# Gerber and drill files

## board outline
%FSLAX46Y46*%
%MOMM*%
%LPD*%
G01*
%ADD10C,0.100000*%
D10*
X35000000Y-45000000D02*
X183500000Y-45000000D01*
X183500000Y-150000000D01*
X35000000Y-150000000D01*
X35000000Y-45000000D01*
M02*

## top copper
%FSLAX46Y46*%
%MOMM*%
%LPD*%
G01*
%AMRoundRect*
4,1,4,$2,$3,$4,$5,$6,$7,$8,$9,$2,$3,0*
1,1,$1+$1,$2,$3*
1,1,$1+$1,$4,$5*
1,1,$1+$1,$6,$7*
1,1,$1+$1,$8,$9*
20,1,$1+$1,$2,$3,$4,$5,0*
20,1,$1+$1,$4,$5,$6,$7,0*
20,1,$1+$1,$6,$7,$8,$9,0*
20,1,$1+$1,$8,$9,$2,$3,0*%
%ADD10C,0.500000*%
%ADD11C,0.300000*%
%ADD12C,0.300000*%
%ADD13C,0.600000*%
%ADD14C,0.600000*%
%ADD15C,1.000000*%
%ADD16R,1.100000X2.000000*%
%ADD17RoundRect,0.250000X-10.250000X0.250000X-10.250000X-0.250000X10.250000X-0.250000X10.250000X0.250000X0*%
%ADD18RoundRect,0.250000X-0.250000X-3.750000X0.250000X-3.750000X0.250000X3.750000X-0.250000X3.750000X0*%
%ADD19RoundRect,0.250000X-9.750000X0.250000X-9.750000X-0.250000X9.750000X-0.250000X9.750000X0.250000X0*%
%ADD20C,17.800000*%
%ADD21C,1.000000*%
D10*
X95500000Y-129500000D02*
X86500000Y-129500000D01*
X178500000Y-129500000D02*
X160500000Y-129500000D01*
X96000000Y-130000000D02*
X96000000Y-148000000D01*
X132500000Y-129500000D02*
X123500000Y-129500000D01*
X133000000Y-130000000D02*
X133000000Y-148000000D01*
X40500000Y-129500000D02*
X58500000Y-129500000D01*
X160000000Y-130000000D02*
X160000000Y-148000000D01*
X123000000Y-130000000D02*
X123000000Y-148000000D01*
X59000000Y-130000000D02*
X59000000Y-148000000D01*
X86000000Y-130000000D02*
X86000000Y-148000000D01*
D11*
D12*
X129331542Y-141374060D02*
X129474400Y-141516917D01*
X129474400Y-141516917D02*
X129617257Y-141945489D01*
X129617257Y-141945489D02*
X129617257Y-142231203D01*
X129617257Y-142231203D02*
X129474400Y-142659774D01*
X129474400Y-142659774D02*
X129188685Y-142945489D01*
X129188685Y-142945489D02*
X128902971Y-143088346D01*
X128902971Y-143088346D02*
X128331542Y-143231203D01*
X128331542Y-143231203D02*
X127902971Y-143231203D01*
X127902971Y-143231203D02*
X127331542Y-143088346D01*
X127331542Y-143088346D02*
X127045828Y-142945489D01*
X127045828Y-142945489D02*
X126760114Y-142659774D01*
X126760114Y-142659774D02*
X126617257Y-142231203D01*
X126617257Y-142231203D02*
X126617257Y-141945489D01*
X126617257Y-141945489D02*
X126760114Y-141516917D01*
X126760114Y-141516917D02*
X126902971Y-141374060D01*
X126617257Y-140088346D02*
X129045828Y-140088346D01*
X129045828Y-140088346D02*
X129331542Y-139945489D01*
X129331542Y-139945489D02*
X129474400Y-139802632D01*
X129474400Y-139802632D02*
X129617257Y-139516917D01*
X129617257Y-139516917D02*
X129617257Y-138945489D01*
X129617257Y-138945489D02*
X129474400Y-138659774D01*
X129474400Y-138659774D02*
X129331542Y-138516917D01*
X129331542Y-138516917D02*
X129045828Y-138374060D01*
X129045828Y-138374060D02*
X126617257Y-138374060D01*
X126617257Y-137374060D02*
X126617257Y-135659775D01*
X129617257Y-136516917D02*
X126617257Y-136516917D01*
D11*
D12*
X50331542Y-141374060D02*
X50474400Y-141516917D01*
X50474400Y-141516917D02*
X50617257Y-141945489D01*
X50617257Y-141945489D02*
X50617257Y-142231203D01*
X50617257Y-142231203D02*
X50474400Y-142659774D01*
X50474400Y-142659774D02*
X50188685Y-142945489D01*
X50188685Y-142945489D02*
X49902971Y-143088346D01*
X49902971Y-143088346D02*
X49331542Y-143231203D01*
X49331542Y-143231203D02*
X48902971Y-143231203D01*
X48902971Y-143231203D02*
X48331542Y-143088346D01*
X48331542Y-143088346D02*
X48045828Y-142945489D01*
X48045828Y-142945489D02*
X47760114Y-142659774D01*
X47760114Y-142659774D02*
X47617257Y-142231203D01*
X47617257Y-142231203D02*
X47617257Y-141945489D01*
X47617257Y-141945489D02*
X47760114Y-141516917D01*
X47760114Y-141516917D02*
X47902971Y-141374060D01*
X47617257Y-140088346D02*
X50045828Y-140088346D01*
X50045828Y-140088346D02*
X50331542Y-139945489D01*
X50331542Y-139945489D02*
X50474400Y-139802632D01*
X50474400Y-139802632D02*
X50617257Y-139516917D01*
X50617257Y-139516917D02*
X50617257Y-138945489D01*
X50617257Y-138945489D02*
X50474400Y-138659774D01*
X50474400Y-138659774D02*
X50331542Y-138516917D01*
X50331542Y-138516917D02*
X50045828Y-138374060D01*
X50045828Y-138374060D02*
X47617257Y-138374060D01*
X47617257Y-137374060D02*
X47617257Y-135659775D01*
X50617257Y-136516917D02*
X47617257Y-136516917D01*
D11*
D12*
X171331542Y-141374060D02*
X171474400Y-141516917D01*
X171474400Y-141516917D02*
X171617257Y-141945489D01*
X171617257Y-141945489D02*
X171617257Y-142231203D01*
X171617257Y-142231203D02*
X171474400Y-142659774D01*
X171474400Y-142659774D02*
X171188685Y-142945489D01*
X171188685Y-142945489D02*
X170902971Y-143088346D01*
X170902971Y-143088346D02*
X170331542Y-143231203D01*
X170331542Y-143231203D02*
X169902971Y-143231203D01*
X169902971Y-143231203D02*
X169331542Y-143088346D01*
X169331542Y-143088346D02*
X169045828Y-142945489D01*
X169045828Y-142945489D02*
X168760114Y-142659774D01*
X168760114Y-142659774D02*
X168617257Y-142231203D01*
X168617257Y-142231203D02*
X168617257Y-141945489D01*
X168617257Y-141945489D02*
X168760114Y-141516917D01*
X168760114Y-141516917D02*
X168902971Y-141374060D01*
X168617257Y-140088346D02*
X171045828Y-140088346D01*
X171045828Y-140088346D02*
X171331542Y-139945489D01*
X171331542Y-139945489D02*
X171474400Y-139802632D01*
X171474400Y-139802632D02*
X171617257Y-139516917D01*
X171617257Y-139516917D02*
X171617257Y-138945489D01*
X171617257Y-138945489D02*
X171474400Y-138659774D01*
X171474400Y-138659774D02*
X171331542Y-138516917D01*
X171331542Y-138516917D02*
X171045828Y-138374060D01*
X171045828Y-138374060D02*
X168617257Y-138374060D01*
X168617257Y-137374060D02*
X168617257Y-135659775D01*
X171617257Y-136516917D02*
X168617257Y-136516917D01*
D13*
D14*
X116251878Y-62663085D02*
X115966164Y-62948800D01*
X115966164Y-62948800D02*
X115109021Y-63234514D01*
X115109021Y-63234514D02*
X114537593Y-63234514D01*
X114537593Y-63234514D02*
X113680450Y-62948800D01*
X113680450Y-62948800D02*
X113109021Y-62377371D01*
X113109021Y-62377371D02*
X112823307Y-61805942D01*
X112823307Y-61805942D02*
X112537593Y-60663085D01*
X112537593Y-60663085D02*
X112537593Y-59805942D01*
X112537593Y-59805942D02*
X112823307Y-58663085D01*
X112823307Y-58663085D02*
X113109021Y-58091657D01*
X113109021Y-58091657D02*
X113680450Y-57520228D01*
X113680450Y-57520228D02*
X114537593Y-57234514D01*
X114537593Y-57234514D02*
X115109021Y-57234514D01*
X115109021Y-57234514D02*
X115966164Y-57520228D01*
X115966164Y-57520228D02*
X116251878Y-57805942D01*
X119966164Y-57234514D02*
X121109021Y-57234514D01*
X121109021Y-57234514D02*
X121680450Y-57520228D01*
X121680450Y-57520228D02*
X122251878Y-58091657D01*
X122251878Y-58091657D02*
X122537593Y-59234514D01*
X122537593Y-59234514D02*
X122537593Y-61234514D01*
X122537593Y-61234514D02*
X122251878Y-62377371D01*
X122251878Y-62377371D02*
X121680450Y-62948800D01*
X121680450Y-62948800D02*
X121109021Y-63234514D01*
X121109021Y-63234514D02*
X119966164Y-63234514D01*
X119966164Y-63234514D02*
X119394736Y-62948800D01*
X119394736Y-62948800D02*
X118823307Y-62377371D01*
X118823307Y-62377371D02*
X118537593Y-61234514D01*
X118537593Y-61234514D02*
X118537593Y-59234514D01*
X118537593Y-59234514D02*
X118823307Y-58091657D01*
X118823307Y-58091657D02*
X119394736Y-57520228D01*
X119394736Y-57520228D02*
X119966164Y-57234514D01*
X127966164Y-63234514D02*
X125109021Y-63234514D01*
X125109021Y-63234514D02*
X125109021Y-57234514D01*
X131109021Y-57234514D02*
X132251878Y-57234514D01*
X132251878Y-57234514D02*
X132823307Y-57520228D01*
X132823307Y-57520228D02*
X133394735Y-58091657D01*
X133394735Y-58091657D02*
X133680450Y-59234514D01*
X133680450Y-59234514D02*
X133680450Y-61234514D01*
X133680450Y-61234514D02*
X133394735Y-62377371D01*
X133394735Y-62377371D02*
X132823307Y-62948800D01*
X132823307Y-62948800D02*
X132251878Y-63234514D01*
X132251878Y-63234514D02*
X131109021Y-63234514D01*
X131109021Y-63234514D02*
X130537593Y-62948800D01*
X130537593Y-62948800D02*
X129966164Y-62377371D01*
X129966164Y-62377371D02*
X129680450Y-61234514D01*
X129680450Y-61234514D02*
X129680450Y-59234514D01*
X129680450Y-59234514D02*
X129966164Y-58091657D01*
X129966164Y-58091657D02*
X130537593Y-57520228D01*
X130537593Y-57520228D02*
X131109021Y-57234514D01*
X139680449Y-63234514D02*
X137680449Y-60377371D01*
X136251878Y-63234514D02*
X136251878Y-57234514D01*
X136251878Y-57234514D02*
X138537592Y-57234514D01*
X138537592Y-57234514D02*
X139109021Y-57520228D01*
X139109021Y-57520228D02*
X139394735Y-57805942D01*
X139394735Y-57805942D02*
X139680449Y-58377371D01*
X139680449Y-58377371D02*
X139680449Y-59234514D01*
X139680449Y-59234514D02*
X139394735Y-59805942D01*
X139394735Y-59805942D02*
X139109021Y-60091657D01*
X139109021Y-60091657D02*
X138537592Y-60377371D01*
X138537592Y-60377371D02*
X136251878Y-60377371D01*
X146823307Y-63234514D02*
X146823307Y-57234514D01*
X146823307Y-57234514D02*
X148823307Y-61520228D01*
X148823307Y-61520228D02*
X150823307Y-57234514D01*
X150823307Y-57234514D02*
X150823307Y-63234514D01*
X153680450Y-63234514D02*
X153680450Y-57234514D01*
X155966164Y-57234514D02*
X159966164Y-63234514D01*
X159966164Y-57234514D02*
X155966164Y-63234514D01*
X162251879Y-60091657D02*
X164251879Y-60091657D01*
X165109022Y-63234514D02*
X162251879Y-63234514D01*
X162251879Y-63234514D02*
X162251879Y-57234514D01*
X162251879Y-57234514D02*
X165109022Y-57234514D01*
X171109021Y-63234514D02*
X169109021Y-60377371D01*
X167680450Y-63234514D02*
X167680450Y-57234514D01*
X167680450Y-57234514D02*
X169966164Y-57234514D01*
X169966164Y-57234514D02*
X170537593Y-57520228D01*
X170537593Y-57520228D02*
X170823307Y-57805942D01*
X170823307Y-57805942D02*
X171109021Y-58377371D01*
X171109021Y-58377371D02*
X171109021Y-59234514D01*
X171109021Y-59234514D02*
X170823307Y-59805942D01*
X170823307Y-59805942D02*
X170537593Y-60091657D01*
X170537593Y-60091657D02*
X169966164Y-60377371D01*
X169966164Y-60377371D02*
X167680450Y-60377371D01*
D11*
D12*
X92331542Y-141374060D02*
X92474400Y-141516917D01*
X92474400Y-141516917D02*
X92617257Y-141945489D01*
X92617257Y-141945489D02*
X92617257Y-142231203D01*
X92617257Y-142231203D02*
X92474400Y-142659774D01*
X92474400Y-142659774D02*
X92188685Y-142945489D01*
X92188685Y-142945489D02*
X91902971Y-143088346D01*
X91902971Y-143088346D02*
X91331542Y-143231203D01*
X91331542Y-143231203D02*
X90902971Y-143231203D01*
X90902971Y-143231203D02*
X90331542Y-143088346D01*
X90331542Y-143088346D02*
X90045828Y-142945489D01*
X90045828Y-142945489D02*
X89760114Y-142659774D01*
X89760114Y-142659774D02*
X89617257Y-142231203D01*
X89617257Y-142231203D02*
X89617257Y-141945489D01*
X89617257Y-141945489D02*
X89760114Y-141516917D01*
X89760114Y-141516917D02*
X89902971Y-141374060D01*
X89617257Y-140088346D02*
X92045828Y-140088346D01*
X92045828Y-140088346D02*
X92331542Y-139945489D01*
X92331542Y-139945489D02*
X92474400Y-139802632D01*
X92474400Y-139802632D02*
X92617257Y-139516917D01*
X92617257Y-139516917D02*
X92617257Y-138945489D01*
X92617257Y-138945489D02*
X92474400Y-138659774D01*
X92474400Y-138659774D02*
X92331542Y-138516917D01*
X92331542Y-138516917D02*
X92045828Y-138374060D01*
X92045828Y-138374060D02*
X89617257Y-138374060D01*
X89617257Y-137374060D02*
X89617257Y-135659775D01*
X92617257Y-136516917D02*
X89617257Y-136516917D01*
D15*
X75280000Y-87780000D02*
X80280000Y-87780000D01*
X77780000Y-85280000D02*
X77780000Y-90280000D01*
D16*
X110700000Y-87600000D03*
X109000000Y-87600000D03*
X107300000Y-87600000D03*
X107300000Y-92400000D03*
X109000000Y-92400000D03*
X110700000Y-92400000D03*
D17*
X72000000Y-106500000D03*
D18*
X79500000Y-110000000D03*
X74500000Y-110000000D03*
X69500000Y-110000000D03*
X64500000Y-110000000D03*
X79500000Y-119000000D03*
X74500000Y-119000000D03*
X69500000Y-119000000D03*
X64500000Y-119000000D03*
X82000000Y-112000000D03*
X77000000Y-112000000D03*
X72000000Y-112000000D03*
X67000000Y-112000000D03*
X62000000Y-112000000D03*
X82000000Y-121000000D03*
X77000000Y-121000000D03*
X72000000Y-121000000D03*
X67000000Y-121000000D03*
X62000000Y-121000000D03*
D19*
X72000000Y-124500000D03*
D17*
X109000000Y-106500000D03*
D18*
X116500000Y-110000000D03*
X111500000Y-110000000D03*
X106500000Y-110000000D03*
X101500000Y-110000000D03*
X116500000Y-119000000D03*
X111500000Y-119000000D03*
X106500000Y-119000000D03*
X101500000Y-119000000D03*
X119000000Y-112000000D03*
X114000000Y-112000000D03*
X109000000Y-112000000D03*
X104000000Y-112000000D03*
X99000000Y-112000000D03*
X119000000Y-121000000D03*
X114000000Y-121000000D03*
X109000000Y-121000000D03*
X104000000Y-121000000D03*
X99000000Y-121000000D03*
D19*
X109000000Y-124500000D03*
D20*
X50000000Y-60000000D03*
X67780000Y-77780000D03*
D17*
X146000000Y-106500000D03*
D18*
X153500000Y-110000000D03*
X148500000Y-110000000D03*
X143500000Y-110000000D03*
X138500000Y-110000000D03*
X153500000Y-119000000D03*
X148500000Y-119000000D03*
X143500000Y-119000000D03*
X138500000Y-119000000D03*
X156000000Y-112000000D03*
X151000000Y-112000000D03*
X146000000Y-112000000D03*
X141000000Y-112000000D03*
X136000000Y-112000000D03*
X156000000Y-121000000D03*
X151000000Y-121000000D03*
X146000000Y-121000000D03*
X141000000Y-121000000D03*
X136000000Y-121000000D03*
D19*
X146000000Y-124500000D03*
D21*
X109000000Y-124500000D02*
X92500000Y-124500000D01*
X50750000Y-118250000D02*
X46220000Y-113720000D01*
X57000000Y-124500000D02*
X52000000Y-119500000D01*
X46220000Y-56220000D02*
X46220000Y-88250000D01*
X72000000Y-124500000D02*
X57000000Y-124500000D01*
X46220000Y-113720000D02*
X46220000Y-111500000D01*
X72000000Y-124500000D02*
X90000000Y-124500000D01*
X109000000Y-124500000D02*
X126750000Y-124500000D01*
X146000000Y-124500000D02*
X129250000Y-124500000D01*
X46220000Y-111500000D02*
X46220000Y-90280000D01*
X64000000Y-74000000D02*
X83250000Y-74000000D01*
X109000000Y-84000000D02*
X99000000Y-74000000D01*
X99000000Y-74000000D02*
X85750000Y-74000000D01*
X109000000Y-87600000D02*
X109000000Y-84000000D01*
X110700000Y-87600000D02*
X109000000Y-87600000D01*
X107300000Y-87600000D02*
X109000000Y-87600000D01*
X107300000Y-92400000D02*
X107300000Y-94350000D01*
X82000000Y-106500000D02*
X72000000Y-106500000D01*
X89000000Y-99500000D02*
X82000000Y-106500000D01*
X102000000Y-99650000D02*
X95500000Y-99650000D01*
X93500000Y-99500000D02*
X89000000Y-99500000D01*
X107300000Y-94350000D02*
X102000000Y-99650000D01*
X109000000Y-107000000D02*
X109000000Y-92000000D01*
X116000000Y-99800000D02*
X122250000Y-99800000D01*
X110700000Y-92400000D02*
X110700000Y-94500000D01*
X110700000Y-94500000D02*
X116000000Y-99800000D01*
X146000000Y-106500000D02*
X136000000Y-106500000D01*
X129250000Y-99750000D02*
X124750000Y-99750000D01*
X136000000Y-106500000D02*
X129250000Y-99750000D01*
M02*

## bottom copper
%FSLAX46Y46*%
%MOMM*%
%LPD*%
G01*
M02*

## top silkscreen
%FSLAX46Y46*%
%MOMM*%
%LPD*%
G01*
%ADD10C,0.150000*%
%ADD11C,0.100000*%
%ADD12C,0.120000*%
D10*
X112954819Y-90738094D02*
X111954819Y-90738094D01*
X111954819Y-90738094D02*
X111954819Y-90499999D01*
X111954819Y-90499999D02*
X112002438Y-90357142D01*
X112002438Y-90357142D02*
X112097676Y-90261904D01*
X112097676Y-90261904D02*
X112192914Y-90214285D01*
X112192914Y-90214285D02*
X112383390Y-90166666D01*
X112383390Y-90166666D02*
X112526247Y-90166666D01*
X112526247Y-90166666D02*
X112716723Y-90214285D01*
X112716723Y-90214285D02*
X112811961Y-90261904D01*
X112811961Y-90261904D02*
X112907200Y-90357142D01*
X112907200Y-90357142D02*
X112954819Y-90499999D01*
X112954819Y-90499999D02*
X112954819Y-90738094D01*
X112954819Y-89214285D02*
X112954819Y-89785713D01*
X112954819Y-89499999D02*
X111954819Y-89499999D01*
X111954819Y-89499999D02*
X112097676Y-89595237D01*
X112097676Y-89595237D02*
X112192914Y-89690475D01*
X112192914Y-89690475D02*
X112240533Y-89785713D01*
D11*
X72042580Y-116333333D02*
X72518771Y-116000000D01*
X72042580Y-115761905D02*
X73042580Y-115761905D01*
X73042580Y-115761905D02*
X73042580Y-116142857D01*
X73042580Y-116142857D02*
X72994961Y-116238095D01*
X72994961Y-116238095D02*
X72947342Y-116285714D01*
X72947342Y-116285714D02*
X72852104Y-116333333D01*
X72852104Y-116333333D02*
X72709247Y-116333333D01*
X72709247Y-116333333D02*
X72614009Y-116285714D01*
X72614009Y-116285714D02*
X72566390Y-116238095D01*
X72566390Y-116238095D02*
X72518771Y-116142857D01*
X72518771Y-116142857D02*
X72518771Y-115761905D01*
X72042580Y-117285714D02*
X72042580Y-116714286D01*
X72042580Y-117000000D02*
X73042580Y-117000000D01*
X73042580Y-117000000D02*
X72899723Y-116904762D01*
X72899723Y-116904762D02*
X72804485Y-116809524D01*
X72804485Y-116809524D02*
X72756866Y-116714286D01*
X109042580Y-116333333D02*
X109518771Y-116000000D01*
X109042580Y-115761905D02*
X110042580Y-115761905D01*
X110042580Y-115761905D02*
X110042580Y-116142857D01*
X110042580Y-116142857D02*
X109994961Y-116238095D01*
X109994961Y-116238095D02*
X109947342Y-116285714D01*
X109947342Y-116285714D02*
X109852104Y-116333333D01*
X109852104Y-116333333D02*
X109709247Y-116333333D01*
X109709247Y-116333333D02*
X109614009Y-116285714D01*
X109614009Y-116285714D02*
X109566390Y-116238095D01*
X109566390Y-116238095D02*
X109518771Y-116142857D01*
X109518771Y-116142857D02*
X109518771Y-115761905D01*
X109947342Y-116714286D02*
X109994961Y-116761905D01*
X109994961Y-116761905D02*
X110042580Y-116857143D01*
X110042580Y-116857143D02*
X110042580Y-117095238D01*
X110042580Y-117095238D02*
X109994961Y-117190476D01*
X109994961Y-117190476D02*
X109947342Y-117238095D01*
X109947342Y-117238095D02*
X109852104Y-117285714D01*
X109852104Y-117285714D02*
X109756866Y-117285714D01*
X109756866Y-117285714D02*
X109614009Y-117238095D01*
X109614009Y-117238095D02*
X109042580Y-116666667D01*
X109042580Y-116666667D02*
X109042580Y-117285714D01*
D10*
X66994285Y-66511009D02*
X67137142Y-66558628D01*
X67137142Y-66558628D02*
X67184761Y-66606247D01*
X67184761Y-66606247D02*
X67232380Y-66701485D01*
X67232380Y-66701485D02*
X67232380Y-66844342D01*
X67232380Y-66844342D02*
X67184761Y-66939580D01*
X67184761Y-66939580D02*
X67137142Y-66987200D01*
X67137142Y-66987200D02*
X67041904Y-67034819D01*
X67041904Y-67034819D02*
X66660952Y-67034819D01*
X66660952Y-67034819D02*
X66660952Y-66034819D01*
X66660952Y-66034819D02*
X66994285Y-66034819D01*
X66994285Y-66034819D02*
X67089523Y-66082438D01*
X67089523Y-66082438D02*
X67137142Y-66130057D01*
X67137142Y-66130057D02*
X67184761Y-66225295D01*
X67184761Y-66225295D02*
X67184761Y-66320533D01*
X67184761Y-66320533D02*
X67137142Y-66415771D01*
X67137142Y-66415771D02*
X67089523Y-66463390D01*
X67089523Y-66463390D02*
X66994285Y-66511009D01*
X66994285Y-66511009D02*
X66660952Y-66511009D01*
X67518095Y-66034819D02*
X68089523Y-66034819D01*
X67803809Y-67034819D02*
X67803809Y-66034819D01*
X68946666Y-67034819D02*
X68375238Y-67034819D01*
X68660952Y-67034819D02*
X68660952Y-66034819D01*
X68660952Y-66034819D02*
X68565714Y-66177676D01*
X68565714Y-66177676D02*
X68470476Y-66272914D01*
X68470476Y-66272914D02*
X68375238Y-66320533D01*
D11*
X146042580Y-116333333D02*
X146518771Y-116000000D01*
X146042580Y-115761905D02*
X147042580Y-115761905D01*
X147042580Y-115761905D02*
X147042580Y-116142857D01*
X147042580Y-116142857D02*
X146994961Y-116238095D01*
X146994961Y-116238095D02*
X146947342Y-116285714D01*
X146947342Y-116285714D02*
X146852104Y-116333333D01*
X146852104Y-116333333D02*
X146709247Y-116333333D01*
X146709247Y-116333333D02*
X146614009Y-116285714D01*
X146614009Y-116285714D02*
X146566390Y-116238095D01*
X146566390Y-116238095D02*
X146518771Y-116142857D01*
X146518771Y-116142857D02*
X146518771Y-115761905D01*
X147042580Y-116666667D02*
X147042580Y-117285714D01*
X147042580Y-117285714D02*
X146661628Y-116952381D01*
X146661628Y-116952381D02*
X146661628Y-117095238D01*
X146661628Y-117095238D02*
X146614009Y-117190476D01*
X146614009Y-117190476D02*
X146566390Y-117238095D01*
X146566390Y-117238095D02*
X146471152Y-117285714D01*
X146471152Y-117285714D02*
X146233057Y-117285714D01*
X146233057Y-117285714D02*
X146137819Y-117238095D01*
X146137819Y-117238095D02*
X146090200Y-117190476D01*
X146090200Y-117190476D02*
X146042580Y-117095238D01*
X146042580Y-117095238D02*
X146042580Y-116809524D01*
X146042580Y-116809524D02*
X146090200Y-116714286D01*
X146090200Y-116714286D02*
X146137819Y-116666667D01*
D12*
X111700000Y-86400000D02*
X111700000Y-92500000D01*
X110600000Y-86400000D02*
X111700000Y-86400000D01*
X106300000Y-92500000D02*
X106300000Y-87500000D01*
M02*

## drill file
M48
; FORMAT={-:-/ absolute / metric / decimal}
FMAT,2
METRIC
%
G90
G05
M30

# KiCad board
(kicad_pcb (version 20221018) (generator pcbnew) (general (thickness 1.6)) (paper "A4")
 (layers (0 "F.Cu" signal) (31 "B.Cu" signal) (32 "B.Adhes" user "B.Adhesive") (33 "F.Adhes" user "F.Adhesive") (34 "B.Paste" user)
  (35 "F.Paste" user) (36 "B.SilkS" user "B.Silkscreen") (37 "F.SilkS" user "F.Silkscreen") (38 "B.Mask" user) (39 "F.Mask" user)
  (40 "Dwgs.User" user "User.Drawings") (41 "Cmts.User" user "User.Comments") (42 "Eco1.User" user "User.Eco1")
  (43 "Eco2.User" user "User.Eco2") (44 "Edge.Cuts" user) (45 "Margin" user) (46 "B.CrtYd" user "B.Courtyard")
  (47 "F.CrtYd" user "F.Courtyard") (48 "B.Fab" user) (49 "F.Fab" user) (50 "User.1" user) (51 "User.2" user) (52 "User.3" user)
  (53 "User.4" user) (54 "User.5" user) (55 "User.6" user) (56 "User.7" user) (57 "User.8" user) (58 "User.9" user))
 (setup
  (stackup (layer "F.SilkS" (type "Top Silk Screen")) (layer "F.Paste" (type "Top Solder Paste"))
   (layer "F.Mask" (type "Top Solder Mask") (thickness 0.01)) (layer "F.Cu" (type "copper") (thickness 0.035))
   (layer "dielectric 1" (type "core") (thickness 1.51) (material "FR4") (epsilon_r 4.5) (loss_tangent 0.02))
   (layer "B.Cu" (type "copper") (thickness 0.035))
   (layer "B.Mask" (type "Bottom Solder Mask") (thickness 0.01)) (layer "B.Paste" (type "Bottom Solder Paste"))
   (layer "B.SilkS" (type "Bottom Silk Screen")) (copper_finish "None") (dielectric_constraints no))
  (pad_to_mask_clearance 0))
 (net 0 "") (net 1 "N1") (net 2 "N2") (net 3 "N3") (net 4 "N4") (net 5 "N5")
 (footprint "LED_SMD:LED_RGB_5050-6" (layer "F.Cu") (at 109 90 -90)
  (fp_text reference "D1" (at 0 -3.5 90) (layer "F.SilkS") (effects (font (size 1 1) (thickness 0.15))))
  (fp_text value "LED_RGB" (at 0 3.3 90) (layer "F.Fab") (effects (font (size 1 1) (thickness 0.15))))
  (fp_line (start -3.6 -2.7) (end 2.5 -2.7) (stroke (width 0.12) (type solid)) (layer "F.SilkS"))
  (fp_line (start -3.6 -1.6) (end -3.6 -2.7) (stroke (width 0.12) (type solid)) (layer "F.SilkS"))
  (fp_line (start 2.5 2.7) (end -2.5 2.7) (stroke (width 0.12) (type solid)) (layer "F.SilkS"))
  (pad "1" smd rect (at -2.4 -1.7) (size 1.1 2) (layers "F.Cu" "F.Paste" "F.Mask") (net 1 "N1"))
  (pad "2" smd rect (at -2.4 0) (size 1.1 2) (layers "F.Cu" "F.Paste" "F.Mask") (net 1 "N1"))
  (pad "3" smd rect (at -2.4 1.7) (size 1.1 2) (layers "F.Cu" "F.Paste" "F.Mask") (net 1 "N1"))
  (pad "4" smd rect (at 2.4 1.7) (size 1.1 2) (layers "F.Cu" "F.Paste" "F.Mask") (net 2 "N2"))
  (pad "5" smd rect (at 2.4 0) (size 1.1 2) (layers "F.Cu" "F.Paste" "F.Mask") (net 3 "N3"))
  (pad "6" smd rect (at 2.4 -1.7) (size 1.1 2) (layers "F.Cu" "F.Paste" "F.Mask") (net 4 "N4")))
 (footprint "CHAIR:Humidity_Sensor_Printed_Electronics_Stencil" (layer "F.Cu") (at 72 116.5 -90)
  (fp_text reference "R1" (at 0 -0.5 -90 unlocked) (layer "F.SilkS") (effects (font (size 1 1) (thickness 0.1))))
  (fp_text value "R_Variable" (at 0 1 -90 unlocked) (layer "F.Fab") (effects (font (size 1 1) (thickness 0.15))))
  (pad "1" smd roundrect (at -10 0 270) (size 1 21) (layers "F.Cu" "F.Paste" "F.Mask") (roundrect_rratio 0.25) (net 2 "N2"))
  (pad "1" smd roundrect (at -6.5 -7.5) (size 1 8) (layers "F.Cu" "F.Paste" "F.Mask") (roundrect_rratio 0.25) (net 2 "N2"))
  (pad "1" smd roundrect (at -6.5 -2.5) (size 1 8) (layers "F.Cu" "F.Paste" "F.Mask") (roundrect_rratio 0.25) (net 2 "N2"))
  (pad "1" smd roundrect (at -6.5 2.5) (size 1 8) (layers "F.Cu" "F.Paste" "F.Mask") (roundrect_rratio 0.25) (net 2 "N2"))
  (pad "1" smd roundrect (at -6.5 7.5) (size 1 8) (layers "F.Cu" "F.Paste" "F.Mask") (roundrect_rratio 0.25) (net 2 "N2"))
  (pad "1" smd roundrect (at 2.5 -7.5) (size 1 8) (layers "F.Cu" "F.Paste" "F.Mask") (roundrect_rratio 0.25) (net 2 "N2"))
  (pad "1" smd roundrect (at 2.5 -2.5) (size 1 8) (layers "F.Cu" "F.Paste" "F.Mask") (roundrect_rratio 0.25) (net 2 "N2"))
  (pad "1" smd roundrect (at 2.5 2.5) (size 1 8) (layers "F.Cu" "F.Paste" "F.Mask") (roundrect_rratio 0.25) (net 2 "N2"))
  (pad "1" smd roundrect (at 2.5 7.5) (size 1 8) (layers "F.Cu" "F.Paste" "F.Mask") (roundrect_rratio 0.25) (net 2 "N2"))
  (pad "2" smd roundrect (at -4.5 -10) (size 1 8) (layers "F.Cu" "F.Paste" "F.Mask") (roundrect_rratio 0.25) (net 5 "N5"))
  (pad "2" smd roundrect (at -4.5 -5) (size 1 8) (layers "F.Cu" "F.Paste" "F.Mask") (roundrect_rratio 0.25) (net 5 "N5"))
  (pad "2" smd roundrect (at -4.5 0) (size 1 8) (layers "F.Cu" "F.Paste" "F.Mask") (roundrect_rratio 0.25) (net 5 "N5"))
  (pad "2" smd roundrect (at -4.5 5) (size 1 8) (layers "F.Cu" "F.Paste" "F.Mask") (roundrect_rratio 0.25) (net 5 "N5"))
  (pad "2" smd roundrect (at -4.5 10) (size 1 8) (layers "F.Cu" "F.Paste" "F.Mask") (roundrect_rratio 0.25) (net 5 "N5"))
  (pad "2" smd roundrect (at 4.5 -10) (size 1 8) (layers "F.Cu" "F.Paste" "F.Mask") (roundrect_rratio 0.25) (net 5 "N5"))
  (pad "2" smd roundrect (at 4.5 -5) (size 1 8) (layers "F.Cu" "F.Paste" "F.Mask") (roundrect_rratio 0.25) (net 5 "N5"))
  (pad "2" smd roundrect (at 4.5 0) (size 1 8) (layers "F.Cu" "F.Paste" "F.Mask") (roundrect_rratio 0.25) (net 5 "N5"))
  (pad "2" smd roundrect (at 4.5 5) (size 1 8) (layers "F.Cu" "F.Paste" "F.Mask") (roundrect_rratio 0.25) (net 5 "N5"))
  (pad "2" smd roundrect (at 4.5 10) (size 1 8) (layers "F.Cu" "F.Paste" "F.Mask") (roundrect_rratio 0.25) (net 5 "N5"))
  (pad "2" smd roundrect (at 8 0 270) (size 1 20) (layers "F.Cu" "F.Paste" "F.Mask") (roundrect_rratio 0.25) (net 5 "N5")))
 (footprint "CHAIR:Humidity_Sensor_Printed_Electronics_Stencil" (layer "F.Cu") (at 109 116.5 -90)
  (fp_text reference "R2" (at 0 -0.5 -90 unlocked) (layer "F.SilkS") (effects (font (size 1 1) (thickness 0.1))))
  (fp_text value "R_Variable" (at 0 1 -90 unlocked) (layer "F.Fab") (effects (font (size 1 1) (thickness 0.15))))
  (pad "1" smd roundrect (at -10 0 270) (size 1 21) (layers "F.Cu" "F.Paste" "F.Mask") (roundrect_rratio 0.25) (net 3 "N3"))
  (pad "1" smd roundrect (at -6.5 -7.5) (size 1 8) (layers "F.Cu" "F.Paste" "F.Mask") (roundrect_rratio 0.25) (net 3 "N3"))
  (pad "1" smd roundrect (at -6.5 -2.5) (size 1 8) (layers "F.Cu" "F.Paste" "F.Mask") (roundrect_rratio 0.25) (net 3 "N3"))
  (pad "1" smd roundrect (at -6.5 2.5) (size 1 8) (layers "F.Cu" "F.Paste" "F.Mask") (roundrect_rratio 0.25) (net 3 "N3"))
  (pad "1" smd roundrect (at -6.5 7.5) (size 1 8) (layers "F.Cu" "F.Paste" "F.Mask") (roundrect_rratio 0.25) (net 3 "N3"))
  (pad "1" smd roundrect (at 2.5 -7.5) (size 1 8) (layers "F.Cu" "F.Paste" "F.Mask") (roundrect_rratio 0.25) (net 3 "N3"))
  (pad "1" smd roundrect (at 2.5 -2.5) (size 1 8) (layers "F.Cu" "F.Paste" "F.Mask") (roundrect_rratio 0.25) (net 3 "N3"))
  (pad "1" smd roundrect (at 2.5 2.5) (size 1 8) (layers "F.Cu" "F.Paste" "F.Mask") (roundrect_rratio 0.25) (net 3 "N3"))
  (pad "1" smd roundrect (at 2.5 7.5) (size 1 8) (layers "F.Cu" "F.Paste" "F.Mask") (roundrect_rratio 0.25) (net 3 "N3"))
  (pad "2" smd roundrect (at -4.5 -10) (size 1 8) (layers "F.Cu" "F.Paste" "F.Mask") (roundrect_rratio 0.25) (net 5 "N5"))
  (pad "2" smd roundrect (at -4.5 -5) (size 1 8) (layers "F.Cu" "F.Paste" "F.Mask") (roundrect_rratio 0.25) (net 5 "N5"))
  (pad "2" smd roundrect (at -4.5 0) (size 1 8) (layers "F.Cu" "F.Paste" "F.Mask") (roundrect_rratio 0.25) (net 5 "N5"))
  (pad "2" smd roundrect (at -4.5 5) (size 1 8) (layers "F.Cu" "F.Paste" "F.Mask") (roundrect_rratio 0.25) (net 5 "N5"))
  (pad "2" smd roundrect (at -4.5 10) (size 1 8) (layers "F.Cu" "F.Paste" "F.Mask") (roundrect_rratio 0.25) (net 5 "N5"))
  (pad "2" smd roundrect (at 4.5 -10) (size 1 8) (layers "F.Cu" "F.Paste" "F.Mask") (roundrect_rratio 0.25) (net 5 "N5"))
  (pad "2" smd roundrect (at 4.5 -5) (size 1 8) (layers "F.Cu" "F.Paste" "F.Mask") (roundrect_rratio 0.25) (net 5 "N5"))
  (pad "2" smd roundrect (at 4.5 0) (size 1 8) (layers "F.Cu" "F.Paste" "F.Mask") (roundrect_rratio 0.25) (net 5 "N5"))
  (pad "2" smd roundrect (at 4.5 5) (size 1 8) (layers "F.Cu" "F.Paste" "F.Mask") (roundrect_rratio 0.25) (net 5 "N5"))
  (pad "2" smd roundrect (at 4.5 10) (size 1 8) (layers "F.Cu" "F.Paste" "F.Mask") (roundrect_rratio 0.25) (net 5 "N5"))
  (pad "2" smd roundrect (at 8 0 270) (size 1 20) (layers "F.Cu" "F.Paste" "F.Mask") (roundrect_rratio 0.25) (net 5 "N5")))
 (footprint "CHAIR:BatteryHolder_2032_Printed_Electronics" (layer "F.Cu") (at 67.78 77.78)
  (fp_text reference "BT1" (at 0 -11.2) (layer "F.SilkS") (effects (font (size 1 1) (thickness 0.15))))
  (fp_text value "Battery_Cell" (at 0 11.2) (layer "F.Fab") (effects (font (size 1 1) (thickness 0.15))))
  (fp_line (start 7.5 10) (end 12.5 10) (stroke (width 1) (type default)) (layer "F.Cu"))
  (fp_line (start 10 7.5) (end 10 12.5) (stroke (width 1) (type default)) (layer "F.Cu"))
  (pad "1" smd circle (at -17.78 -17.78) (size 17.8 17.8) (layers "F.Cu" "F.Mask") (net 5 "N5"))
  (pad "2" smd circle (at 0 0) (size 17.8 17.8) (layers "F.Cu" "F.Mask") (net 1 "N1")))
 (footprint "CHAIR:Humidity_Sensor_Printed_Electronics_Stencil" (layer "F.Cu") (at 146 116.5 -90)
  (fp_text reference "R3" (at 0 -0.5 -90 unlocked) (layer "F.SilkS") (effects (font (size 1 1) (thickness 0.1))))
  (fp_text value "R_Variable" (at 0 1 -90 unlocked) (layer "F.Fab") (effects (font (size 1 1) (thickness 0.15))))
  (pad "1" smd roundrect (at -10 0 270) (size 1 21) (layers "F.Cu" "F.Paste" "F.Mask") (roundrect_rratio 0.25) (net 4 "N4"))
  (pad "1" smd roundrect (at -6.5 -7.5) (size 1 8) (layers "F.Cu" "F.Paste" "F.Mask") (roundrect_rratio 0.25) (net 4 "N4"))
  (pad "1" smd roundrect (at -6.5 -2.5) (size 1 8) (layers "F.Cu" "F.Paste" "F.Mask") (roundrect_rratio 0.25) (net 4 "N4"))
  (pad "1" smd roundrect (at -6.5 2.5) (size 1 8) (layers "F.Cu" "F.Paste" "F.Mask") (roundrect_rratio 0.25) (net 4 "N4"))
  (pad "1" smd roundrect (at -6.5 7.5) (size 1 8) (layers "F.Cu" "F.Paste" "F.Mask") (roundrect_rratio 0.25) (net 4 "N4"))
  (pad "1" smd roundrect (at 2.5 -7.5) (size 1 8) (layers "F.Cu" "F.Paste" "F.Mask") (roundrect_rratio 0.25) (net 4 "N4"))
  (pad "1" smd roundrect (at 2.5 -2.5) (size 1 8) (layers "F.Cu" "F.Paste" "F.Mask") (roundrect_rratio 0.25) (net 4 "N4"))
  (pad "1" smd roundrect (at 2.5 2.5) (size 1 8) (layers "F.Cu" "F.Paste" "F.Mask") (roundrect_rratio 0.25) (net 4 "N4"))
  (pad "1" smd roundrect (at 2.5 7.5) (size 1 8) (layers "F.Cu" "F.Paste" "F.Mask") (roundrect_rratio 0.25) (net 4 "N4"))
  (pad "2" smd roundrect (at -4.5 -10) (size 1 8) (layers "F.Cu" "F.Paste" "F.Mask") (roundrect_rratio 0.25) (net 5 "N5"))
  (pad "2" smd roundrect (at -4.5 -5) (size 1 8) (layers "F.Cu" "F.Paste" "F.Mask") (roundrect_rratio 0.25) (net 5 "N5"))
  (pad "2" smd roundrect (at -4.5 0) (size 1 8) (layers "F.Cu" "F.Paste" "F.Mask") (roundrect_rratio 0.25) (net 5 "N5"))
  (pad "2" smd roundrect (at -4.5 5) (size 1 8) (layers "F.Cu" "F.Paste" "F.Mask") (roundrect_rratio 0.25) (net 5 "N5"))
  (pad "2" smd roundrect (at -4.5 10) (size 1 8) (layers "F.Cu" "F.Paste" "F.Mask") (roundrect_rratio 0.25) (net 5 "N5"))
  (pad "2" smd roundrect (at 4.5 -10) (size 1 8) (layers "F.Cu" "F.Paste" "F.Mask") (roundrect_rratio 0.25) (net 5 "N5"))
  (pad "2" smd roundrect (at 4.5 -5) (size 1 8) (layers "F.Cu" "F.Paste" "F.Mask") (roundrect_rratio 0.25) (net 5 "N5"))
  (pad "2" smd roundrect (at 4.5 0) (size 1 8) (layers "F.Cu" "F.Paste" "F.Mask") (roundrect_rratio 0.25) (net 5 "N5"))
  (pad "2" smd roundrect (at 4.5 5) (size 1 8) (layers "F.Cu" "F.Paste" "F.Mask") (roundrect_rratio 0.25) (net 5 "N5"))
  (pad "2" smd roundrect (at 4.5 10) (size 1 8) (layers "F.Cu" "F.Paste" "F.Mask") (roundrect_rratio 0.25) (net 5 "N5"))
  (pad "2" smd roundrect (at 8 0 270) (size 1 20) (layers "F.Cu" "F.Paste" "F.Mask") (roundrect_rratio 0.25) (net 5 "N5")))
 (gr_line (start 95.5 129.5) (end 86.5 129.5) (stroke (width 0.5) (type default)) (layer "F.Cu"))
 (gr_line (start 178.5 129.5) (end 160.5 129.5) (stroke (width 0.5) (type default)) (layer "F.Cu"))
 (gr_line (start 96 130) (end 96 148) (stroke (width 0.5) (type default)) (layer "F.Cu"))
 (gr_line (start 132.5 129.5) (end 123.5 129.5) (stroke (width 0.5) (type default)) (layer "F.Cu"))
 (gr_line (start 133 130) (end 133 148) (stroke (width 0.5) (type default)) (layer "F.Cu"))
 (gr_line (start 40.5 129.5) (end 58.5 129.5) (stroke (width 0.5) (type default)) (layer "F.Cu"))
 (gr_line (start 160 130) (end 160 148) (stroke (width 0.5) (type default)) (layer "F.Cu"))
 (gr_line (start 123 130) (end 123 148) (stroke (width 0.5) (type default)) (layer "F.Cu"))
 (gr_line (start 59 130) (end 59 148) (stroke (width 0.5) (type default)) (layer "F.Cu"))
 (gr_line (start 86 130) (end 86 148) (stroke (width 0.5) (type default)) (layer "F.Cu"))
 (gr_rect (start 35 45) (end 183.5 150) (stroke (width 0.1) (type default)) (fill none) (layer "Edge.Cuts"))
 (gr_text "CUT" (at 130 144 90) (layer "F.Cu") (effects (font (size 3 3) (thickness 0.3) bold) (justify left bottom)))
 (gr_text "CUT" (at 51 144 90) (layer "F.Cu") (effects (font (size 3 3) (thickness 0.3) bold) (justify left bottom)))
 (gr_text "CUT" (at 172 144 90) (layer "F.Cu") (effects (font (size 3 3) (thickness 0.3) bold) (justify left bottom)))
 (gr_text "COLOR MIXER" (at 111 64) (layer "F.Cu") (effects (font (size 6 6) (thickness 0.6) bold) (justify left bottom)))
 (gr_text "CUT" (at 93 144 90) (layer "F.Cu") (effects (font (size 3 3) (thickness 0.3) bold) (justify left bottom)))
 (segment (start 109 124.5) (end 92.5 124.5) (width 1) (layer "F.Cu") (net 5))
 (segment (start 50.75 118.25) (end 46.22 113.72) (width 1) (layer "F.Cu") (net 5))
 (segment (start 57 124.5) (end 52 119.5) (width 1) (layer "F.Cu") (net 5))
 (segment (start 46.22 56.22) (end 46.22 88.25) (width 1) (layer "F.Cu") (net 5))
 (segment (start 72 124.5) (end 57 124.5) (width 1) (layer "F.Cu") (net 5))
 (segment (start 46.22 113.72) (end 46.22 111.5) (width 1) (layer "F.Cu") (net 5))
 (segment (start 72 124.5) (end 90 124.5) (width 1) (layer "F.Cu") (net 5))
 (segment (start 109 124.5) (end 126.75 124.5) (width 1) (layer "F.Cu") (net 5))
 (segment (start 146 124.5) (end 129.25 124.5) (width 1) (layer "F.Cu") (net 5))
 (segment (start 46.22 111.5) (end 46.22 90.28) (width 1) (layer "F.Cu") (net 5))
 (segment (start 64 74) (end 83.25 74) (width 1) (layer "F.Cu") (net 1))
 (segment (start 109 84) (end 99 74) (width 1) (layer "F.Cu") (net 1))
 (segment (start 99 74) (end 85.75 74) (width 1) (layer "F.Cu") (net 1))
 (segment (start 109 87.6) (end 109 84) (width 1) (layer "F.Cu") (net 1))
 (segment (start 110.7 87.6) (end 109 87.6) (width 1) (layer "F.Cu") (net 1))
 (segment (start 107.3 87.6) (end 109 87.6) (width 1) (layer "F.Cu") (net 1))
 (segment (start 107.3 92.4) (end 107.3 94.35) (width 1) (layer "F.Cu") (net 2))
 (segment (start 82 106.5) (end 72 106.5) (width 1) (layer "F.Cu") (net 2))
 (segment (start 89 99.5) (end 82 106.5) (width 1) (layer "F.Cu") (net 2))
 (segment (start 102 99.65) (end 95.5 99.65) (width 1) (layer "F.Cu") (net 2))
 (segment (start 93.5 99.5) (end 89 99.5) (width 1) (layer "F.Cu") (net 2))
 (segment (start 107.3 94.35) (end 102 99.65) (width 1) (layer "F.Cu") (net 2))
 (segment (start 109 107) (end 109 92) (width 1) (layer "F.Cu") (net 3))
 (segment (start 116 99.8) (end 122.25 99.8) (width 1) (layer "F.Cu") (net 4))
 (segment (start 110.7 92.4) (end 110.7 94.5) (width 1) (layer "F.Cu") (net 4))
 (segment (start 110.7 94.5) (end 116 99.8) (width 1) (layer "F.Cu") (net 4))
 (segment (start 146 106.5) (end 136 106.5) (width 1) (layer "F.Cu") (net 4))
 (segment (start 129.25 99.75) (end 124.75 99.75) (width 1) (layer "F.Cu") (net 4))
 (segment (start 136 106.5) (end 129.25 99.75) (width 1) (layer "F.Cu") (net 4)))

